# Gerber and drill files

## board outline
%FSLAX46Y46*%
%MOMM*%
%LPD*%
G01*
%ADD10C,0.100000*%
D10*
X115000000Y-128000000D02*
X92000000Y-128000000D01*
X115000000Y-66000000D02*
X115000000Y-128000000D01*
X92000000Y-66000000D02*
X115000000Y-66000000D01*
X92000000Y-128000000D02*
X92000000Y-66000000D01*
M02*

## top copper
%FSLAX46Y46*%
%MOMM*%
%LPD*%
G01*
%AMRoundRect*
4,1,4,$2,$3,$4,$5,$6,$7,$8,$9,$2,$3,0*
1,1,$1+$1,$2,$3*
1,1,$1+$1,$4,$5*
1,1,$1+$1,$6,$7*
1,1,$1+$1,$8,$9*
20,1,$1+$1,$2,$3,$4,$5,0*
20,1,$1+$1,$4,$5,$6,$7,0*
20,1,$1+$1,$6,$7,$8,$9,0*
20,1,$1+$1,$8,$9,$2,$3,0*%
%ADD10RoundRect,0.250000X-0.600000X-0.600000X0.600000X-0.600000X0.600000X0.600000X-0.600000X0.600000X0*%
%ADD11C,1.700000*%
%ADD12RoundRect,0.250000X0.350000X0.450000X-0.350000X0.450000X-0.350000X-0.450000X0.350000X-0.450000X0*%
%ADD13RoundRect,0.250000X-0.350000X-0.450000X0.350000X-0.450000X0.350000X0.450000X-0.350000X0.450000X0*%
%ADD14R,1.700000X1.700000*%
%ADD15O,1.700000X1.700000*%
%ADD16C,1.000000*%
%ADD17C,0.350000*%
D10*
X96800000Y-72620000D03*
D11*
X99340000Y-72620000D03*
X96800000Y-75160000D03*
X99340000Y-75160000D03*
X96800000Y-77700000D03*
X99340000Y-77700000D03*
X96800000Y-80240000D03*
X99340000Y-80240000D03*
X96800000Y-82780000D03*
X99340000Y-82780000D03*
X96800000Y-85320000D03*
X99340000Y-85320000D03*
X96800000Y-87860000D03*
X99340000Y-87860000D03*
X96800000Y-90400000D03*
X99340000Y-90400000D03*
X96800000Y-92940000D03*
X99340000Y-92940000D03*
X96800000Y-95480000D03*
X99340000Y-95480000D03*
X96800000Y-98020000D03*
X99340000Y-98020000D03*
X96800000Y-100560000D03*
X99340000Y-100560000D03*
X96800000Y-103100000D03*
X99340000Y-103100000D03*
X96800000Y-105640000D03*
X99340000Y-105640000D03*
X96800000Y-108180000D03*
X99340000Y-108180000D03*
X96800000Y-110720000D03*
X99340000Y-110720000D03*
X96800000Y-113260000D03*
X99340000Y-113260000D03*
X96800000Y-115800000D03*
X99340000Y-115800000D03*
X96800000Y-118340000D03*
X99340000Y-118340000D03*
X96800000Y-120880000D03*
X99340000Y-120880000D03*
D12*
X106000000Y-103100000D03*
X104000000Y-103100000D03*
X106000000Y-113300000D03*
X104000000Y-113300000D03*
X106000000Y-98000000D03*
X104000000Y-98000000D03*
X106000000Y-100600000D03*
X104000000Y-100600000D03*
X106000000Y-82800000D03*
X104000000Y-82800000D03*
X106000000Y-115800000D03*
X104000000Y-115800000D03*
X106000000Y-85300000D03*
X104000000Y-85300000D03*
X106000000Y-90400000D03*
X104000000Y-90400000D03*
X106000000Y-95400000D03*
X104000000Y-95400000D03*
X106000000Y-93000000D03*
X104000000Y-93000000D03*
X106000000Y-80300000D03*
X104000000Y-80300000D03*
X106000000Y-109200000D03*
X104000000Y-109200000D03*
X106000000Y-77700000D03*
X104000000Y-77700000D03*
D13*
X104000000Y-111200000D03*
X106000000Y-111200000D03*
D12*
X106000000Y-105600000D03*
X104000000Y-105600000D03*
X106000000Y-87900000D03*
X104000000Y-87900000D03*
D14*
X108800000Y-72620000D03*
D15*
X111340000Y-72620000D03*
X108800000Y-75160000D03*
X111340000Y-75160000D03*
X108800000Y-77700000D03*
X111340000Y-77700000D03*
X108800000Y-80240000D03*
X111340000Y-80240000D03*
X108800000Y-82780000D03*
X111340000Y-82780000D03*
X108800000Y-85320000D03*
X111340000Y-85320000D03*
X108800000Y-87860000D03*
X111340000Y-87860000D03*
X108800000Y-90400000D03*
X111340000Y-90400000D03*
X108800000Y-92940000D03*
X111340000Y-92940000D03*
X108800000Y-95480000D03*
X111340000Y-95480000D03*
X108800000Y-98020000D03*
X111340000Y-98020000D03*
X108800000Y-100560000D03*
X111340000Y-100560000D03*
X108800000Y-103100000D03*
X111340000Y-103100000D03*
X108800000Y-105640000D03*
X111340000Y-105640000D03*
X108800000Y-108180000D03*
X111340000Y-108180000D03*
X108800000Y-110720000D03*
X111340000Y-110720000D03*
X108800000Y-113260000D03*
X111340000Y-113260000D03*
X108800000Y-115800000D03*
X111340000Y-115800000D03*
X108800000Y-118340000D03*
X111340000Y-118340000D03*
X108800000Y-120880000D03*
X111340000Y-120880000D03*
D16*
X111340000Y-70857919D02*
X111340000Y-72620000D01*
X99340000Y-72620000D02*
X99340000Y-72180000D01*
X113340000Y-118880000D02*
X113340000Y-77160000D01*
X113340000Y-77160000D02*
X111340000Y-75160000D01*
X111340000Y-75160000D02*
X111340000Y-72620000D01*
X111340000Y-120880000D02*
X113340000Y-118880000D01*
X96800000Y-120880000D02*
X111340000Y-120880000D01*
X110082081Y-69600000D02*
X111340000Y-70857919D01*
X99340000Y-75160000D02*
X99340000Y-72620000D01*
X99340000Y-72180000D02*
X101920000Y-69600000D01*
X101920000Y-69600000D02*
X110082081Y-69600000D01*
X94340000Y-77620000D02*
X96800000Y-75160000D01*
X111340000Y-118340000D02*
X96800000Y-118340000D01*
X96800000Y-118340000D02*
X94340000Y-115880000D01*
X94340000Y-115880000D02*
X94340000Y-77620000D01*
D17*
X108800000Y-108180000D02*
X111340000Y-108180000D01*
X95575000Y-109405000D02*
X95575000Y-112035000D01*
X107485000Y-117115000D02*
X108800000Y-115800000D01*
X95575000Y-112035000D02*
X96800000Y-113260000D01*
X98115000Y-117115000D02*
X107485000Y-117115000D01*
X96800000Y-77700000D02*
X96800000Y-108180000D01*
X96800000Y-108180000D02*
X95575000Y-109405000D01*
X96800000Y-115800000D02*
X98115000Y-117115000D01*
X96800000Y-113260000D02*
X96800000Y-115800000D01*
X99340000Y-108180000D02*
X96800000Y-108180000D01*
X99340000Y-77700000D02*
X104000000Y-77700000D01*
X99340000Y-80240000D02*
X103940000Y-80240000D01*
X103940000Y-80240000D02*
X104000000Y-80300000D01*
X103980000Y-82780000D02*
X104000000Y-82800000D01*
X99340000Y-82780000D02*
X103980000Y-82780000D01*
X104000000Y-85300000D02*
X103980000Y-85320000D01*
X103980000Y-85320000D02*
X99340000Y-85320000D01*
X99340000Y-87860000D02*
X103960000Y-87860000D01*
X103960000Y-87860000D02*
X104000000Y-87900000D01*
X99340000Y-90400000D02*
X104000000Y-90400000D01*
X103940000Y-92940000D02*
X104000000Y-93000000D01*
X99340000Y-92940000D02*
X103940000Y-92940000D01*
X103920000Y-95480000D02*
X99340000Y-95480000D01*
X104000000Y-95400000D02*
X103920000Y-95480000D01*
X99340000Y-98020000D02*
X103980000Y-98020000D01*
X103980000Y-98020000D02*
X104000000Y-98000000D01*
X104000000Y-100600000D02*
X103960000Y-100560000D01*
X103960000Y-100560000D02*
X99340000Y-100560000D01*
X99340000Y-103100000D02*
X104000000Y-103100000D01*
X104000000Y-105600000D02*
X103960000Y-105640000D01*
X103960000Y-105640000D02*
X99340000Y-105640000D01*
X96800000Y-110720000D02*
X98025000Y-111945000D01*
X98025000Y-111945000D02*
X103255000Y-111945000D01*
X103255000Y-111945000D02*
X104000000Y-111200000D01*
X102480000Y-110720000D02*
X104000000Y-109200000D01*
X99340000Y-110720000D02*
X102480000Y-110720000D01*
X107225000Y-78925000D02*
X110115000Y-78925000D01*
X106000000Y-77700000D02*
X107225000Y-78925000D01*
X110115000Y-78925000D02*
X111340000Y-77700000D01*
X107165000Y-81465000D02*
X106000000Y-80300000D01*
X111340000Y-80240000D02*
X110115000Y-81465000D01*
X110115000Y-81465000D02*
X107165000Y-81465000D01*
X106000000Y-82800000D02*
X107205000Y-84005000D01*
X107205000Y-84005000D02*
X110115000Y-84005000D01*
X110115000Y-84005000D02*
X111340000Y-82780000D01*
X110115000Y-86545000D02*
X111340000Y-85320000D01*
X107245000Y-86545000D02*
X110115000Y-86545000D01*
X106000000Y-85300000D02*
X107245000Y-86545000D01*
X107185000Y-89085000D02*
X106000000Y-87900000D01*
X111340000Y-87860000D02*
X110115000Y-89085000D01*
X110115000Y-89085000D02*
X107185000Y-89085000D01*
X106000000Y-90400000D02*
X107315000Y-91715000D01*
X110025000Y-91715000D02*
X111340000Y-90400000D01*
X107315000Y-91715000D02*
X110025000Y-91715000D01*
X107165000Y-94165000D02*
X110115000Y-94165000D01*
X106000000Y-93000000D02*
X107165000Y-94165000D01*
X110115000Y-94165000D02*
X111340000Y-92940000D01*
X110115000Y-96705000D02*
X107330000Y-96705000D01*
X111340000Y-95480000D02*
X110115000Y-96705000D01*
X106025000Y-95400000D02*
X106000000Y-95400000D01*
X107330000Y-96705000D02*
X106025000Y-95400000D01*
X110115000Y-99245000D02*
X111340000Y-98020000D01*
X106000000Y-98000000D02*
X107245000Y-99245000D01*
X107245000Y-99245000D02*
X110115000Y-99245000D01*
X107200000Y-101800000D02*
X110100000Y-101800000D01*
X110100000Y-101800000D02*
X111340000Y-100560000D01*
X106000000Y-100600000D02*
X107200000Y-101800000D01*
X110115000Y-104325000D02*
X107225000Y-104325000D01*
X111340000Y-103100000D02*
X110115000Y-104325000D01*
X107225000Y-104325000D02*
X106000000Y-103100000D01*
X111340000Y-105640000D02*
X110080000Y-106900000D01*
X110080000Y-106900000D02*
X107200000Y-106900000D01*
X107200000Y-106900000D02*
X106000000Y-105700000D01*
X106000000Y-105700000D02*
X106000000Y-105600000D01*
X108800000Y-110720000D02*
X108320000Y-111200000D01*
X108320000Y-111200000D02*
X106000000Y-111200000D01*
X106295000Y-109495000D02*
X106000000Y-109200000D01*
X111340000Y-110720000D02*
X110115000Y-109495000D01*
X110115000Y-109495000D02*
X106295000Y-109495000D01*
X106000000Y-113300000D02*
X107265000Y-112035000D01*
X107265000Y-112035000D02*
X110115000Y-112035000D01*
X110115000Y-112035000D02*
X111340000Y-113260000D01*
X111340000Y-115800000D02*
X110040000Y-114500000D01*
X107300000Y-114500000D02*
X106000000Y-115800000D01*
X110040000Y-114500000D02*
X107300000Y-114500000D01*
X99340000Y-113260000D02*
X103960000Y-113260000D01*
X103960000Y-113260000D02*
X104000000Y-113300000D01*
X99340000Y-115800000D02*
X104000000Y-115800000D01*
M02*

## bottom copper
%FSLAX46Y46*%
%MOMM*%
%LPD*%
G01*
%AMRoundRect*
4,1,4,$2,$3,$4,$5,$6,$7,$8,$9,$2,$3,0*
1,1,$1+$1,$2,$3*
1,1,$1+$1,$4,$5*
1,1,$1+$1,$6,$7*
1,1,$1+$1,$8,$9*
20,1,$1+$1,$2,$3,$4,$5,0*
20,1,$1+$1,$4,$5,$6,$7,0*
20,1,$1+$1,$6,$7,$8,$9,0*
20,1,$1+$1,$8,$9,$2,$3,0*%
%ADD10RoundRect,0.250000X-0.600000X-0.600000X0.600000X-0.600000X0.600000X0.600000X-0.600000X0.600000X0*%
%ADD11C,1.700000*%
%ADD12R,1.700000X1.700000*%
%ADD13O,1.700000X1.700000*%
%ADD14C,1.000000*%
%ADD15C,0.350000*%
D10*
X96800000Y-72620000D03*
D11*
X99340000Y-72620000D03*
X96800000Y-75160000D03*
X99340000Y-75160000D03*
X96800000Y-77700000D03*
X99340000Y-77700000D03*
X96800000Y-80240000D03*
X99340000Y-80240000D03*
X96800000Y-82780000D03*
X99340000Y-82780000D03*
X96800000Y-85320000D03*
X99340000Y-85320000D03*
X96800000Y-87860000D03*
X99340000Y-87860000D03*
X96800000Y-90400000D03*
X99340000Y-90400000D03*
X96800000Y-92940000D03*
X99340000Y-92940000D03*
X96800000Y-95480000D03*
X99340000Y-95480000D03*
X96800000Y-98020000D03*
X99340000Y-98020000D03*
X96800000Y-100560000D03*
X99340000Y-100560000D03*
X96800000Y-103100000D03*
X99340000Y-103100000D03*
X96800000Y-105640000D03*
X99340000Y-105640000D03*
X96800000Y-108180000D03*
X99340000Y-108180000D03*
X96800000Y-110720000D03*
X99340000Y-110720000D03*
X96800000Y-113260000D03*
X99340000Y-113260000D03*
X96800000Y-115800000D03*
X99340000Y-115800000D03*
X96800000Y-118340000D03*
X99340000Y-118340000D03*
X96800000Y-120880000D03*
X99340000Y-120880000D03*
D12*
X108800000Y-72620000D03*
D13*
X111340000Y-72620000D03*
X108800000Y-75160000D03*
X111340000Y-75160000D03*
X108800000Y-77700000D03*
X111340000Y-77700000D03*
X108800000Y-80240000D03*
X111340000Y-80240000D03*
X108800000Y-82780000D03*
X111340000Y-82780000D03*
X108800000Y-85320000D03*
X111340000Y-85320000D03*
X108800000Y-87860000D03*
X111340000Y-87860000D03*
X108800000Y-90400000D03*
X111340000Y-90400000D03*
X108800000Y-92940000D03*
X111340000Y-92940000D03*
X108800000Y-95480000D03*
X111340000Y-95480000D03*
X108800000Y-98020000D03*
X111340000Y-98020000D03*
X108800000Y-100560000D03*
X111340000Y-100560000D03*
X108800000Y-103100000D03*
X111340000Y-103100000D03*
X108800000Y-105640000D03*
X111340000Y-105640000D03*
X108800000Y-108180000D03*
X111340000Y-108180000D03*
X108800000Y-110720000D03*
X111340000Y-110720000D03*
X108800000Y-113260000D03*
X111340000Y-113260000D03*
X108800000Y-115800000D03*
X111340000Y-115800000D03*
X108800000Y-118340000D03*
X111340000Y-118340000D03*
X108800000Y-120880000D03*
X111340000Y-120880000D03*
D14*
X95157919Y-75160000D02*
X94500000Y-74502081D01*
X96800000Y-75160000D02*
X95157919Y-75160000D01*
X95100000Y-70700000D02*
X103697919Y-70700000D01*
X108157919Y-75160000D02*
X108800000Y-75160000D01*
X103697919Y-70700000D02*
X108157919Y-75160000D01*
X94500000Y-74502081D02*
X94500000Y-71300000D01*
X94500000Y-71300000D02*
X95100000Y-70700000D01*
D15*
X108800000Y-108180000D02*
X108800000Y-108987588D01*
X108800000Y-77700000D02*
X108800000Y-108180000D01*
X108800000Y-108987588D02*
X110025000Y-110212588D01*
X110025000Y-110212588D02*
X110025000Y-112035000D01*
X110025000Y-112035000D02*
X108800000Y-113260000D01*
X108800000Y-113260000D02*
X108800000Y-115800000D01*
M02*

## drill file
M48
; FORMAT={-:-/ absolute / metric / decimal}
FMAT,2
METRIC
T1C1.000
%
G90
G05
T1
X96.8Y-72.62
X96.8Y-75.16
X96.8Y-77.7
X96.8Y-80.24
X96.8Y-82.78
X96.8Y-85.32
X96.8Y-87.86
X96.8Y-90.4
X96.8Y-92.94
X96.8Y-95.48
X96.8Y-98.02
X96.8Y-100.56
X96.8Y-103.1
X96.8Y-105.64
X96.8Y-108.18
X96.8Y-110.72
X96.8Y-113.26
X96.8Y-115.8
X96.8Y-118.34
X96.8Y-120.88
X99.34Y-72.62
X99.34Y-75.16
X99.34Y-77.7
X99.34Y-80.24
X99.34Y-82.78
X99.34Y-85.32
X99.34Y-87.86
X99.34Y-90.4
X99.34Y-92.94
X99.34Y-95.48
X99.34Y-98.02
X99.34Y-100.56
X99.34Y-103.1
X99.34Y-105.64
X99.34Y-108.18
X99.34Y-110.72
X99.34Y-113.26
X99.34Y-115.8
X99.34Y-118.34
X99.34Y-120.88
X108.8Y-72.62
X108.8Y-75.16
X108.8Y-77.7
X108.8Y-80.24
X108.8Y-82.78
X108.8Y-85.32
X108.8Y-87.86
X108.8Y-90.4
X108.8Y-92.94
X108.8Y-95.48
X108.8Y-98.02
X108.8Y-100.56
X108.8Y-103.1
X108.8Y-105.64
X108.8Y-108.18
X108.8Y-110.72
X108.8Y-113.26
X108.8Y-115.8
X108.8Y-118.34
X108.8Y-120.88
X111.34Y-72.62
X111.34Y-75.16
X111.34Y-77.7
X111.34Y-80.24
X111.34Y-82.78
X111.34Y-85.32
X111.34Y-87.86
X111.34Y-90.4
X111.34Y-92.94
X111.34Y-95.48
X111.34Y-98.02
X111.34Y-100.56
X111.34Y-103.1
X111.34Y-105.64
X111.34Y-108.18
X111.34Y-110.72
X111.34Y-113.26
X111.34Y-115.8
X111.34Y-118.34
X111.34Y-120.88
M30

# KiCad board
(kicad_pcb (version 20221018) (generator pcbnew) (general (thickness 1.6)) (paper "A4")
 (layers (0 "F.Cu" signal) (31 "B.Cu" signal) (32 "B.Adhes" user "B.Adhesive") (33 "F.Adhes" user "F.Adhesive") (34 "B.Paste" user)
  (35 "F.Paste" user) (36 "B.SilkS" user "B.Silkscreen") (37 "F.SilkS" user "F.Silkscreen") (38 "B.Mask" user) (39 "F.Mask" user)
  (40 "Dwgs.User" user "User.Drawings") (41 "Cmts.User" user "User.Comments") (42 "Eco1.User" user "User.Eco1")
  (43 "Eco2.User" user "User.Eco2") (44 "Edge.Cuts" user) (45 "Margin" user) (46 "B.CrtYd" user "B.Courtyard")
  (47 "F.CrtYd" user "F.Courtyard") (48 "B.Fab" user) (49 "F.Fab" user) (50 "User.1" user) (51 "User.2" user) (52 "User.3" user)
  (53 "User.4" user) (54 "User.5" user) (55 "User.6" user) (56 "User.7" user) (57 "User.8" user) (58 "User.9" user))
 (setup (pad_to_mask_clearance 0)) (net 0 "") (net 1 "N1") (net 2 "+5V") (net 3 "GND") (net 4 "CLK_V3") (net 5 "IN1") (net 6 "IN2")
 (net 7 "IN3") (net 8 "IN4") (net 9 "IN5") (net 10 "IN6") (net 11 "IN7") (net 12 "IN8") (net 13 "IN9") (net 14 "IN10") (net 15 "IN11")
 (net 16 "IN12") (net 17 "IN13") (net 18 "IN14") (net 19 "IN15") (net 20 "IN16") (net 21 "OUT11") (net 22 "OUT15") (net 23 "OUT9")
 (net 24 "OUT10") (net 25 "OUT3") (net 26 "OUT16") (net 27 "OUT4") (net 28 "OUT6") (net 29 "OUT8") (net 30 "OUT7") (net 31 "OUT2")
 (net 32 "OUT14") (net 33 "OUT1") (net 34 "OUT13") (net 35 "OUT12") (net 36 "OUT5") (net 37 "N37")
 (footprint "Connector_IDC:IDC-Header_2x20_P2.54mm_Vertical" (layer "F.Cu") (at 96.8 72.62)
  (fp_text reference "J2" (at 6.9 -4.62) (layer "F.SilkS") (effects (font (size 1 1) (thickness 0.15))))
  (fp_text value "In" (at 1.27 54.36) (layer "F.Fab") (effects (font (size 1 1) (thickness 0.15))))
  (pad "1" thru_hole roundrect (at 0 0) (size 1.7 1.7) (drill 1) (layers "*.Cu" "*.Mask") (roundrect_rratio 0.1470588235) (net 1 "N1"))
  (pad "2" thru_hole circle (at 2.54 0) (size 1.7 1.7) (drill 1) (layers "*.Cu" "*.Mask") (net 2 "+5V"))
  (pad "3" thru_hole circle (at 0 2.54) (size 1.7 1.7) (drill 1) (layers "*.Cu" "*.Mask") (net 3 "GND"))
  (pad "4" thru_hole circle (at 2.54 2.54) (size 1.7 1.7) (drill 1) (layers "*.Cu" "*.Mask") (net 2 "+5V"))
  (pad "5" thru_hole circle (at 0 5.08) (size 1.7 1.7) (drill 1) (layers "*.Cu" "*.Mask") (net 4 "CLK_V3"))
  (pad "6" thru_hole circle (at 2.54 5.08) (size 1.7 1.7) (drill 1) (layers "*.Cu" "*.Mask") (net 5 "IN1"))
  (pad "7" thru_hole circle (at 0 7.62) (size 1.7 1.7) (drill 1) (layers "*.Cu" "*.Mask") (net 4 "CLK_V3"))
  (pad "8" thru_hole circle (at 2.54 7.62) (size 1.7 1.7) (drill 1) (layers "*.Cu" "*.Mask") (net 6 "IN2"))
  (pad "9" thru_hole circle (at 0 10.16) (size 1.7 1.7) (drill 1) (layers "*.Cu" "*.Mask") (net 4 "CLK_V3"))
  (pad "10" thru_hole circle (at 2.54 10.16) (size 1.7 1.7) (drill 1) (layers "*.Cu" "*.Mask") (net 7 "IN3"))
  (pad "11" thru_hole circle (at 0 12.7) (size 1.7 1.7) (drill 1) (layers "*.Cu" "*.Mask") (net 4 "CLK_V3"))
  (pad "12" thru_hole circle (at 2.54 12.7) (size 1.7 1.7) (drill 1) (layers "*.Cu" "*.Mask") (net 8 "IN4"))
  (pad "13" thru_hole circle (at 0 15.24) (size 1.7 1.7) (drill 1) (layers "*.Cu" "*.Mask") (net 4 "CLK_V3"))
  (pad "14" thru_hole circle (at 2.54 15.24) (size 1.7 1.7) (drill 1) (layers "*.Cu" "*.Mask") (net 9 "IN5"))
  (pad "15" thru_hole circle (at 0 17.78) (size 1.7 1.7) (drill 1) (layers "*.Cu" "*.Mask") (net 4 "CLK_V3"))
  (pad "16" thru_hole circle (at 2.54 17.78) (size 1.7 1.7) (drill 1) (layers "*.Cu" "*.Mask") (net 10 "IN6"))
  (pad "17" thru_hole circle (at 0 20.32) (size 1.7 1.7) (drill 1) (layers "*.Cu" "*.Mask") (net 4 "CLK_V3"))
  (pad "18" thru_hole circle (at 2.54 20.32) (size 1.7 1.7) (drill 1) (layers "*.Cu" "*.Mask") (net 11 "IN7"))
  (pad "19" thru_hole circle (at 0 22.86) (size 1.7 1.7) (drill 1) (layers "*.Cu" "*.Mask") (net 4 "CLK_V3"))
  (pad "20" thru_hole circle (at 2.54 22.86) (size 1.7 1.7) (drill 1) (layers "*.Cu" "*.Mask") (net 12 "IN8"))
  (pad "21" thru_hole circle (at 0 25.4) (size 1.7 1.7) (drill 1) (layers "*.Cu" "*.Mask") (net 4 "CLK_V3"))
  (pad "22" thru_hole circle (at 2.54 25.4) (size 1.7 1.7) (drill 1) (layers "*.Cu" "*.Mask") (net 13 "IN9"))
  (pad "23" thru_hole circle (at 0 27.94) (size 1.7 1.7) (drill 1) (layers "*.Cu" "*.Mask") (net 4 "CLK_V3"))
  (pad "24" thru_hole circle (at 2.54 27.94) (size 1.7 1.7) (drill 1) (layers "*.Cu" "*.Mask") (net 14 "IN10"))
  (pad "25" thru_hole circle (at 0 30.48) (size 1.7 1.7) (drill 1) (layers "*.Cu" "*.Mask") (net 4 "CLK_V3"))
  (pad "26" thru_hole circle (at 2.54 30.48) (size 1.7 1.7) (drill 1) (layers "*.Cu" "*.Mask") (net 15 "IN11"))
  (pad "27" thru_hole circle (at 0 33.02) (size 1.7 1.7) (drill 1) (layers "*.Cu" "*.Mask") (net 4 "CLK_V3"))
  (pad "28" thru_hole circle (at 2.54 33.02) (size 1.7 1.7) (drill 1) (layers "*.Cu" "*.Mask") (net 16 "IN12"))
  (pad "29" thru_hole circle (at 0 35.56) (size 1.7 1.7) (drill 1) (layers "*.Cu" "*.Mask") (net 4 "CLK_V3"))
  (pad "30" thru_hole circle (at 2.54 35.56) (size 1.7 1.7) (drill 1) (layers "*.Cu" "*.Mask") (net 4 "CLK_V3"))
  (pad "31" thru_hole circle (at 0 38.1) (size 1.7 1.7) (drill 1) (layers "*.Cu" "*.Mask") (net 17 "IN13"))
  (pad "32" thru_hole circle (at 2.54 38.1) (size 1.7 1.7) (drill 1) (layers "*.Cu" "*.Mask") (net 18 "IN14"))
  (pad "33" thru_hole circle (at 0 40.64) (size 1.7 1.7) (drill 1) (layers "*.Cu" "*.Mask") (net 4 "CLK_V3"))
  (pad "34" thru_hole circle (at 2.54 40.64) (size 1.7 1.7) (drill 1) (layers "*.Cu" "*.Mask") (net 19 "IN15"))
  (pad "35" thru_hole circle (at 0 43.18) (size 1.7 1.7) (drill 1) (layers "*.Cu" "*.Mask") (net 4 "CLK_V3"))
  (pad "36" thru_hole circle (at 2.54 43.18) (size 1.7 1.7) (drill 1) (layers "*.Cu" "*.Mask") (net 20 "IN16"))
  (pad "37" thru_hole circle (at 0 45.72) (size 1.7 1.7) (drill 1) (layers "*.Cu" "*.Mask") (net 3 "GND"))
  (pad "38" thru_hole circle (at 2.54 45.72) (size 1.7 1.7) (drill 1) (layers "*.Cu" "*.Mask") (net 3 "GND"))
  (pad "39" thru_hole circle (at 0 48.26) (size 1.7 1.7) (drill 1) (layers "*.Cu" "*.Mask") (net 2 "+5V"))
  (pad "40" thru_hole circle (at 2.54 48.26) (size 1.7 1.7) (drill 1) (layers "*.Cu" "*.Mask") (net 2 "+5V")))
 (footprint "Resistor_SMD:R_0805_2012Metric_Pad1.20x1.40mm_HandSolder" (layer "F.Cu") (at 105 103.1 180)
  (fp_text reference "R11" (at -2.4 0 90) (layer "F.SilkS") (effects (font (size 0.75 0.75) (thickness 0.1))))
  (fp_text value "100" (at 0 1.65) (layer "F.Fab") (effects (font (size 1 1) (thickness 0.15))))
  (pad "1" smd roundrect (at -1 0 180) (size 1.2 1.4) (layers "F.Cu" "F.Paste" "F.Mask") (roundrect_rratio 0.2083333333) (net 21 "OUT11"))
  (pad "2" smd roundrect (at 1 0 180) (size 1.2 1.4) (layers "F.Cu" "F.Paste" "F.Mask") (roundrect_rratio 0.2083333333) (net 15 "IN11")))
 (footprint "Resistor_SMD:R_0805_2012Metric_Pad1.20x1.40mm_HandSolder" (layer "F.Cu") (at 105 113.3 180)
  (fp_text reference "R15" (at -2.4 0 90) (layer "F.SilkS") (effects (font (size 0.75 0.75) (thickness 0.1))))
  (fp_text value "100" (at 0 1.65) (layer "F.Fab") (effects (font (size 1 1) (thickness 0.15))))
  (pad "1" smd roundrect (at -1 0 180) (size 1.2 1.4) (layers "F.Cu" "F.Paste" "F.Mask") (roundrect_rratio 0.2083333333) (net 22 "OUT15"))
  (pad "2" smd roundrect (at 1 0 180) (size 1.2 1.4) (layers "F.Cu" "F.Paste" "F.Mask") (roundrect_rratio 0.2083333333) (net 19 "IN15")))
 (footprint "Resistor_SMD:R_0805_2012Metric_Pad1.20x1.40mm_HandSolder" (layer "F.Cu") (at 105 98 180)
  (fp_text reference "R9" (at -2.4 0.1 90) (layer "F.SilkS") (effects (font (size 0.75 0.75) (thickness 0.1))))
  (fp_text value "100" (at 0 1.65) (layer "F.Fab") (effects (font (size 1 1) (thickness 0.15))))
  (pad "1" smd roundrect (at -1 0 180) (size 1.2 1.4) (layers "F.Cu" "F.Paste" "F.Mask") (roundrect_rratio 0.2083333333) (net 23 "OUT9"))
  (pad "2" smd roundrect (at 1 0 180) (size 1.2 1.4) (layers "F.Cu" "F.Paste" "F.Mask") (roundrect_rratio 0.2083333333) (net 13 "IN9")))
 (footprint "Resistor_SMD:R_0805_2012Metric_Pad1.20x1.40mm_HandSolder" (layer "F.Cu") (at 105 100.6 180)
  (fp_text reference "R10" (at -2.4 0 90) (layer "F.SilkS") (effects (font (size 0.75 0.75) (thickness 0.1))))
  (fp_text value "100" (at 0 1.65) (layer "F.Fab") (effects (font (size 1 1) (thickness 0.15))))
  (pad "1" smd roundrect (at -1 0 180) (size 1.2 1.4) (layers "F.Cu" "F.Paste" "F.Mask") (roundrect_rratio 0.2083333333) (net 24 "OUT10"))
  (pad "2" smd roundrect (at 1 0 180) (size 1.2 1.4) (layers "F.Cu" "F.Paste" "F.Mask") (roundrect_rratio 0.2083333333) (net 14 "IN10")))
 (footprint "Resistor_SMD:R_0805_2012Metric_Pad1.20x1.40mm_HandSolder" (layer "F.Cu") (at 105 82.8 180)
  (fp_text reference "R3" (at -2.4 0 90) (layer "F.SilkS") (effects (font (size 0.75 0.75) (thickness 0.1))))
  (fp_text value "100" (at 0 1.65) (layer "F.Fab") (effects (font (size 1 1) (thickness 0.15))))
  (pad "1" smd roundrect (at -1 0 180) (size 1.2 1.4) (layers "F.Cu" "F.Paste" "F.Mask") (roundrect_rratio 0.2083333333) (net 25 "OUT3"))
  (pad "2" smd roundrect (at 1 0 180) (size 1.2 1.4) (layers "F.Cu" "F.Paste" "F.Mask") (roundrect_rratio 0.2083333333) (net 7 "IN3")))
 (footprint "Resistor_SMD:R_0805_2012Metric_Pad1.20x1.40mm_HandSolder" (layer "F.Cu") (at 105 115.8 180)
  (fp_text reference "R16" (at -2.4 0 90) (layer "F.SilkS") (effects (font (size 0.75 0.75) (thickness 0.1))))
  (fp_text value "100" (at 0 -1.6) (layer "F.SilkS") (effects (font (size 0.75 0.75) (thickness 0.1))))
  (pad "1" smd roundrect (at -1 0 180) (size 1.2 1.4) (layers "F.Cu" "F.Paste" "F.Mask") (roundrect_rratio 0.2083333333) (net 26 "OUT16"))
  (pad "2" smd roundrect (at 1 0 180) (size 1.2 1.4) (layers "F.Cu" "F.Paste" "F.Mask") (roundrect_rratio 0.2083333333) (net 20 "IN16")))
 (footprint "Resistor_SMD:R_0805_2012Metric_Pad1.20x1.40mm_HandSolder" (layer "F.Cu") (at 105 85.3 180)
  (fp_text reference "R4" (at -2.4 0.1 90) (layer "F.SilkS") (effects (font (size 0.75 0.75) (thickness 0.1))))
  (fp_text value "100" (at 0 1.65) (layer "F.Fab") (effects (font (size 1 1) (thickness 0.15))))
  (pad "1" smd roundrect (at -1 0 180) (size 1.2 1.4) (layers "F.Cu" "F.Paste" "F.Mask") (roundrect_rratio 0.2083333333) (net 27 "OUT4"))
  (pad "2" smd roundrect (at 1 0 180) (size 1.2 1.4) (layers "F.Cu" "F.Paste" "F.Mask") (roundrect_rratio 0.2083333333) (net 8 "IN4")))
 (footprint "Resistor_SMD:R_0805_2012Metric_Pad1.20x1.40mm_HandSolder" (layer "F.Cu") (at 105 90.4 180)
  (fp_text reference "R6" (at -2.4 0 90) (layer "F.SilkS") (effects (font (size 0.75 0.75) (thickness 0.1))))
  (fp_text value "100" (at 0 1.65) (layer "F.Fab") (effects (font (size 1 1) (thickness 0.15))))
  (pad "1" smd roundrect (at -1 0 180) (size 1.2 1.4) (layers "F.Cu" "F.Paste" "F.Mask") (roundrect_rratio 0.2083333333) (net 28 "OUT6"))
  (pad "2" smd roundrect (at 1 0 180) (size 1.2 1.4) (layers "F.Cu" "F.Paste" "F.Mask") (roundrect_rratio 0.2083333333) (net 10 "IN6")))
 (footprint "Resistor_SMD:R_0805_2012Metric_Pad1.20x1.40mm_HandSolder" (layer "F.Cu") (at 105 95.4 180)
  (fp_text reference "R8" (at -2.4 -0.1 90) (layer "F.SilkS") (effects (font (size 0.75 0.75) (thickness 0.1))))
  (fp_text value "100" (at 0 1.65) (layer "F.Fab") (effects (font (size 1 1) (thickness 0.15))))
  (pad "1" smd roundrect (at -1 0 180) (size 1.2 1.4) (layers "F.Cu" "F.Paste" "F.Mask") (roundrect_rratio 0.2083333333) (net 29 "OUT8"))
  (pad "2" smd roundrect (at 1 0 180) (size 1.2 1.4) (layers "F.Cu" "F.Paste" "F.Mask") (roundrect_rratio 0.2083333333) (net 12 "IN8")))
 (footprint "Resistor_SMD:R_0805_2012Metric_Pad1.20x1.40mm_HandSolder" (layer "F.Cu") (at 105 93 180)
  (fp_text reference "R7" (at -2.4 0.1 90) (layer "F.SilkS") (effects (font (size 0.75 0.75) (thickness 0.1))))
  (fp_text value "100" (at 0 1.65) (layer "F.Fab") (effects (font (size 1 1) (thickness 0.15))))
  (pad "1" smd roundrect (at -1 0 180) (size 1.2 1.4) (layers "F.Cu" "F.Paste" "F.Mask") (roundrect_rratio 0.2083333333) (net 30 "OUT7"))
  (pad "2" smd roundrect (at 1 0 180) (size 1.2 1.4) (layers "F.Cu" "F.Paste" "F.Mask") (roundrect_rratio 0.2083333333) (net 11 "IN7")))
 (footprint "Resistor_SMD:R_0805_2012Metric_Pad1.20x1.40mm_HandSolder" (layer "F.Cu") (at 105 80.3 180)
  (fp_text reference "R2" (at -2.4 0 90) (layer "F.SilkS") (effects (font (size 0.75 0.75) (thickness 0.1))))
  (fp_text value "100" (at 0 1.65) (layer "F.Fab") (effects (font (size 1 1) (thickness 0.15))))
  (pad "1" smd roundrect (at -1 0 180) (size 1.2 1.4) (layers "F.Cu" "F.Paste" "F.Mask") (roundrect_rratio 0.2083333333) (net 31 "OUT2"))
  (pad "2" smd roundrect (at 1 0 180) (size 1.2 1.4) (layers "F.Cu" "F.Paste" "F.Mask") (roundrect_rratio 0.2083333333) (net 6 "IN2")))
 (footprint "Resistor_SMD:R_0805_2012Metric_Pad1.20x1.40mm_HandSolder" (layer "F.Cu") (at 105 109.2 180)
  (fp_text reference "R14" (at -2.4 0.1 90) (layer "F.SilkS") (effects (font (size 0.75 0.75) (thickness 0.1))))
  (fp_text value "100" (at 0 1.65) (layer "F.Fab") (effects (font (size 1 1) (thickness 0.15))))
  (pad "1" smd roundrect (at -1 0 180) (size 1.2 1.4) (layers "F.Cu" "F.Paste" "F.Mask") (roundrect_rratio 0.2083333333) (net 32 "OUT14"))
  (pad "2" smd roundrect (at 1 0 180) (size 1.2 1.4) (layers "F.Cu" "F.Paste" "F.Mask") (roundrect_rratio 0.2083333333) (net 18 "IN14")))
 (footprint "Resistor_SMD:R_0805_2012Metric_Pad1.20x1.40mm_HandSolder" (layer "F.Cu") (at 105 77.7 180)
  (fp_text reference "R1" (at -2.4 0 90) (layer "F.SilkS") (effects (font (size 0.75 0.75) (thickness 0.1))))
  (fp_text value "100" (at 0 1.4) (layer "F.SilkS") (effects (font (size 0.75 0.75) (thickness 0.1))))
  (pad "1" smd roundrect (at -1 0 180) (size 1.2 1.4) (layers "F.Cu" "F.Paste" "F.Mask") (roundrect_rratio 0.2083333333) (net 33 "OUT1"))
  (pad "2" smd roundrect (at 1 0 180) (size 1.2 1.4) (layers "F.Cu" "F.Paste" "F.Mask") (roundrect_rratio 0.2083333333) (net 5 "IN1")))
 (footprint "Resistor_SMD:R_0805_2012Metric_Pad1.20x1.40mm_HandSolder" (layer "F.Cu") (at 105 111.2)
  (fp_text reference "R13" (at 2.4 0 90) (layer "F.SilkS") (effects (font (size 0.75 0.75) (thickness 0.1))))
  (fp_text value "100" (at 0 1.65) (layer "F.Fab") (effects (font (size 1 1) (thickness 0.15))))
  (pad "1" smd roundrect (at -1 0) (size 1.2 1.4) (layers "F.Cu" "F.Paste" "F.Mask") (roundrect_rratio 0.2083333333) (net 17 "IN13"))
  (pad "2" smd roundrect (at 1 0) (size 1.2 1.4) (layers "F.Cu" "F.Paste" "F.Mask") (roundrect_rratio 0.2083333333) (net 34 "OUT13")))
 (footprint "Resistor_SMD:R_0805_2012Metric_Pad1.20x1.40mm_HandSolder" (layer "F.Cu") (at 105 105.6 180)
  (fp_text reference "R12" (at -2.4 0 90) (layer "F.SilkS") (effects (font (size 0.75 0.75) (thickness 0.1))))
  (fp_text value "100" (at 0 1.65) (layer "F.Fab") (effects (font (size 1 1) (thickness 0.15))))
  (pad "1" smd roundrect (at -1 0 180) (size 1.2 1.4) (layers "F.Cu" "F.Paste" "F.Mask") (roundrect_rratio 0.2083333333) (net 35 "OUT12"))
  (pad "2" smd roundrect (at 1 0 180) (size 1.2 1.4) (layers "F.Cu" "F.Paste" "F.Mask") (roundrect_rratio 0.2083333333) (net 16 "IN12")))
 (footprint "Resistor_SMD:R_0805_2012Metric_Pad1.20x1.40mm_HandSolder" (layer "F.Cu") (at 105 87.9 180)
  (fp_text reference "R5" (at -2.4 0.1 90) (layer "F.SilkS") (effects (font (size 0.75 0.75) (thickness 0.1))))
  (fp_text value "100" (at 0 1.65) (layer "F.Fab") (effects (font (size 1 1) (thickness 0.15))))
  (pad "1" smd roundrect (at -1 0 180) (size 1.2 1.4) (layers "F.Cu" "F.Paste" "F.Mask") (roundrect_rratio 0.2083333333) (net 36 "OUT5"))
  (pad "2" smd roundrect (at 1 0 180) (size 1.2 1.4) (layers "F.Cu" "F.Paste" "F.Mask") (roundrect_rratio 0.2083333333) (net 9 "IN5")))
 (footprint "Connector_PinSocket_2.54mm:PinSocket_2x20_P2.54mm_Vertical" (layer "B.Cu") (at 108.8 72.62 180)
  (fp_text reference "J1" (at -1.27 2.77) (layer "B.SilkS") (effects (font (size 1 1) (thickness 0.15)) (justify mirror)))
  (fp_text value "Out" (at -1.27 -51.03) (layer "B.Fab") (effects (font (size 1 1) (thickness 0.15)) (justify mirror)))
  (pad "1" thru_hole rect (at 0 0 180) (size 1.7 1.7) (drill 1) (layers "*.Cu" "*.Mask") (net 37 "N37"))
  (pad "2" thru_hole oval (at -2.54 0 180) (size 1.7 1.7) (drill 1) (layers "*.Cu" "*.Mask") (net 2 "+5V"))
  (pad "3" thru_hole oval (at 0 -2.54 180) (size 1.7 1.7) (drill 1) (layers "*.Cu" "*.Mask") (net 3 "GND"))
  (pad "4" thru_hole oval (at -2.54 -2.54 180) (size 1.7 1.7) (drill 1) (layers "*.Cu" "*.Mask") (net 2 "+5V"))
  (pad "5" thru_hole oval (at 0 -5.08 180) (size 1.7 1.7) (drill 1) (layers "*.Cu" "*.Mask") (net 4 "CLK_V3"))
  (pad "6" thru_hole oval (at -2.54 -5.08 180) (size 1.7 1.7) (drill 1) (layers "*.Cu" "*.Mask") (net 33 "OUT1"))
  (pad "7" thru_hole oval (at 0 -7.62 180) (size 1.7 1.7) (drill 1) (layers "*.Cu" "*.Mask") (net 4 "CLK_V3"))
  (pad "8" thru_hole oval (at -2.54 -7.62 180) (size 1.7 1.7) (drill 1) (layers "*.Cu" "*.Mask") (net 31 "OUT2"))
  (pad "9" thru_hole oval (at 0 -10.16 180) (size 1.7 1.7) (drill 1) (layers "*.Cu" "*.Mask") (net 4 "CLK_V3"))
  (pad "10" thru_hole oval (at -2.54 -10.16 180) (size 1.7 1.7) (drill 1) (layers "*.Cu" "*.Mask") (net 25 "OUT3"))
  (pad "11" thru_hole oval (at 0 -12.7 180) (size 1.7 1.7) (drill 1) (layers "*.Cu" "*.Mask") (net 4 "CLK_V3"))
  (pad "12" thru_hole oval (at -2.54 -12.7 180) (size 1.7 1.7) (drill 1) (layers "*.Cu" "*.Mask") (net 27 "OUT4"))
  (pad "13" thru_hole oval (at 0 -15.24 180) (size 1.7 1.7) (drill 1) (layers "*.Cu" "*.Mask") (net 4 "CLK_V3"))
  (pad "14" thru_hole oval (at -2.54 -15.24 180) (size 1.7 1.7) (drill 1) (layers "*.Cu" "*.Mask") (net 36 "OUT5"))
  (pad "15" thru_hole oval (at 0 -17.78 180) (size 1.7 1.7) (drill 1) (layers "*.Cu" "*.Mask") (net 4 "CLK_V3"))
  (pad "16" thru_hole oval (at -2.54 -17.78 180) (size 1.7 1.7) (drill 1) (layers "*.Cu" "*.Mask") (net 28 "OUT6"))
  (pad "17" thru_hole oval (at 0 -20.32 180) (size 1.7 1.7) (drill 1) (layers "*.Cu" "*.Mask") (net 4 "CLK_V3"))
  (pad "18" thru_hole oval (at -2.54 -20.32 180) (size 1.7 1.7) (drill 1) (layers "*.Cu" "*.Mask") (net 30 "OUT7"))
  (pad "19" thru_hole oval (at 0 -22.86 180) (size 1.7 1.7) (drill 1) (layers "*.Cu" "*.Mask") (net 4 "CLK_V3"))
  (pad "20" thru_hole oval (at -2.54 -22.86 180) (size 1.7 1.7) (drill 1) (layers "*.Cu" "*.Mask") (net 29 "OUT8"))
  (pad "21" thru_hole oval (at 0 -25.4 180) (size 1.7 1.7) (drill 1) (layers "*.Cu" "*.Mask") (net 4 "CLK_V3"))
  (pad "22" thru_hole oval (at -2.54 -25.4 180) (size 1.7 1.7) (drill 1) (layers "*.Cu" "*.Mask") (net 23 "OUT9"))
  (pad "23" thru_hole oval (at 0 -27.94 180) (size 1.7 1.7) (drill 1) (layers "*.Cu" "*.Mask") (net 4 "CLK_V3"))
  (pad "24" thru_hole oval (at -2.54 -27.94 180) (size 1.7 1.7) (drill 1) (layers "*.Cu" "*.Mask") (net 24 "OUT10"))
  (pad "25" thru_hole oval (at 0 -30.48 180) (size 1.7 1.7) (drill 1) (layers "*.Cu" "*.Mask") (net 4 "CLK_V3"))
  (pad "26" thru_hole oval (at -2.54 -30.48 180) (size 1.7 1.7) (drill 1) (layers "*.Cu" "*.Mask") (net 21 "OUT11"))
  (pad "27" thru_hole oval (at 0 -33.02 180) (size 1.7 1.7) (drill 1) (layers "*.Cu" "*.Mask") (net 4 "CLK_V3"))
  (pad "28" thru_hole oval (at -2.54 -33.02 180) (size 1.7 1.7) (drill 1) (layers "*.Cu" "*.Mask") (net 35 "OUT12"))
  (pad "29" thru_hole oval (at 0 -35.56 180) (size 1.7 1.7) (drill 1) (layers "*.Cu" "*.Mask") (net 4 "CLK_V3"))
  (pad "30" thru_hole oval (at -2.54 -35.56 180) (size 1.7 1.7) (drill 1) (layers "*.Cu" "*.Mask") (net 4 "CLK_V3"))
  (pad "31" thru_hole oval (at 0 -38.1 180) (size 1.7 1.7) (drill 1) (layers "*.Cu" "*.Mask") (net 34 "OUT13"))
  (pad "32" thru_hole oval (at -2.54 -38.1 180) (size 1.7 1.7) (drill 1) (layers "*.Cu" "*.Mask") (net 32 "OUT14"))
  (pad "33" thru_hole oval (at 0 -40.64 180) (size 1.7 1.7) (drill 1) (layers "*.Cu" "*.Mask") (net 4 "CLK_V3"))
  (pad "34" thru_hole oval (at -2.54 -40.64 180) (size 1.7 1.7) (drill 1) (layers "*.Cu" "*.Mask") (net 22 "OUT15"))
  (pad "35" thru_hole oval (at 0 -43.18 180) (size 1.7 1.7) (drill 1) (layers "*.Cu" "*.Mask") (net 4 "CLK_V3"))
  (pad "36" thru_hole oval (at -2.54 -43.18 180) (size 1.7 1.7) (drill 1) (layers "*.Cu" "*.Mask") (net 26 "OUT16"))
  (pad "37" thru_hole oval (at 0 -45.72 180) (size 1.7 1.7) (drill 1) (layers "*.Cu" "*.Mask") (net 3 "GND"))
  (pad "38" thru_hole oval (at -2.54 -45.72 180) (size 1.7 1.7) (drill 1) (layers "*.Cu" "*.Mask") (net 3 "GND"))
  (pad "39" thru_hole oval (at 0 -48.26 180) (size 1.7 1.7) (drill 1) (layers "*.Cu" "*.Mask") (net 2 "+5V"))
  (pad "40" thru_hole oval (at -2.54 -48.26 180) (size 1.7 1.7) (drill 1) (layers "*.Cu" "*.Mask") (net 2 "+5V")))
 (gr_line (start 115 128) (end 92 128) (stroke (width 0.1) (type default)) (layer "Edge.Cuts"))
 (gr_line (start 115 66) (end 115 128) (stroke (width 0.1) (type default)) (layer "Edge.Cuts"))
 (gr_line (start 92 66) (end 115 66) (stroke (width 0.1) (type default)) (layer "Edge.Cuts"))
 (gr_line (start 92 128) (end 92 66) (stroke (width 0.1) (type default)) (layer "Edge.Cuts"))
 (segment (start 111.34 70.857919) (end 111.34 72.62) (width 1) (layer "F.Cu") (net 2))
 (segment (start 99.34 72.62) (end 99.34 72.18) (width 1) (layer "F.Cu") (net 2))
 (segment (start 113.34 118.88) (end 113.34 77.16) (width 1) (layer "F.Cu") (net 2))
 (segment (start 113.34 77.16) (end 111.34 75.16) (width 1) (layer "F.Cu") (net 2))
 (segment (start 111.34 75.16) (end 111.34 72.62) (width 1) (layer "F.Cu") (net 2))
 (segment (start 111.34 120.88) (end 113.34 118.88) (width 1) (layer "F.Cu") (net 2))
 (segment (start 96.8 120.88) (end 111.34 120.88) (width 1) (layer "F.Cu") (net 2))
 (segment (start 110.082081 69.6) (end 111.34 70.857919) (width 1) (layer "F.Cu") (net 2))
 (segment (start 99.34 75.16) (end 99.34 72.62) (width 1) (layer "F.Cu") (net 2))
 (segment (start 99.34 72.18) (end 101.92 69.6) (width 1) (layer "F.Cu") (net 2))
 (segment (start 101.92 69.6) (end 110.082081 69.6) (width 1) (layer "F.Cu") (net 2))
 (segment (start 94.34 77.62) (end 96.8 75.16) (width 1) (layer "F.Cu") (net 3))
 (segment (start 111.34 118.34) (end 96.8 118.34) (width 1) (layer "F.Cu") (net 3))
 (segment (start 96.8 118.34) (end 94.34 115.88) (width 1) (layer "F.Cu") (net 3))
 (segment (start 94.34 115.88) (end 94.34 77.62) (width 1) (layer "F.Cu") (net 3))
 (segment (start 95.157919 75.16) (end 94.5 74.502081) (width 1) (layer "B.Cu") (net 3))
 (segment (start 96.8 75.16) (end 95.157919 75.16) (width 1) (layer "B.Cu") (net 3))
 (segment (start 95.1 70.7) (end 103.697919 70.7) (width 1) (layer "B.Cu") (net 3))
 (segment (start 108.157919 75.16) (end 108.8 75.16) (width 1) (layer "B.Cu") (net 3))
 (segment (start 103.697919 70.7) (end 108.157919 75.16) (width 1) (layer "B.Cu") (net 3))
 (segment (start 94.5 74.502081) (end 94.5 71.3) (width 1) (layer "B.Cu") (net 3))
 (segment (start 94.5 71.3) (end 95.1 70.7) (width 1) (layer "B.Cu") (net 3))
 (segment (start 108.8 108.18) (end 111.34 108.18) (width 0.35) (layer "F.Cu") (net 4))
 (segment (start 95.575 109.405) (end 95.575 112.035) (width 0.35) (layer "F.Cu") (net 4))
 (segment (start 107.485 117.115) (end 108.8 115.8) (width 0.35) (layer "F.Cu") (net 4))
 (segment (start 95.575 112.035) (end 96.8 113.26) (width 0.35) (layer "F.Cu") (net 4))
 (segment (start 98.115 117.115) (end 107.485 117.115) (width 0.35) (layer "F.Cu") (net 4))
 (segment (start 96.8 77.7) (end 96.8 108.18) (width 0.35) (layer "F.Cu") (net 4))
 (segment (start 96.8 108.18) (end 95.575 109.405) (width 0.35) (layer "F.Cu") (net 4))
 (segment (start 96.8 115.8) (end 98.115 117.115) (width 0.35) (layer "F.Cu") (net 4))
 (segment (start 96.8 113.26) (end 96.8 115.8) (width 0.35) (layer "F.Cu") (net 4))
 (segment (start 99.34 108.18) (end 96.8 108.18) (width 0.35) (layer "F.Cu") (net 4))
 (segment (start 108.8 108.18) (end 108.8 108.987588) (width 0.35) (layer "B.Cu") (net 4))
 (segment (start 108.8 77.7) (end 108.8 108.18) (width 0.35) (layer "B.Cu") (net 4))
 (segment (start 108.8 108.987588) (end 110.025 110.212588) (width 0.35) (layer "B.Cu") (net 4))
 (segment (start 110.025 110.212588) (end 110.025 112.035) (width 0.35) (layer "B.Cu") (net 4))
 (segment (start 110.025 112.035) (end 108.8 113.26) (width 0.35) (layer "B.Cu") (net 4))
 (segment (start 108.8 113.26) (end 108.8 115.8) (width 0.35) (layer "B.Cu") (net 4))
 (segment (start 99.34 77.7) (end 104 77.7) (width 0.35) (layer "F.Cu") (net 5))
 (segment (start 99.34 80.24) (end 103.94 80.24) (width 0.35) (layer "F.Cu") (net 6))
 (segment (start 103.94 80.24) (end 104 80.3) (width 0.35) (layer "F.Cu") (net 6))
 (segment (start 103.98 82.78) (end 104 82.8) (width 0.35) (layer "F.Cu") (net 7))
 (segment (start 99.34 82.78) (end 103.98 82.78) (width 0.35) (layer "F.Cu") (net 7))
 (segment (start 104 85.3) (end 103.98 85.32) (width 0.35) (layer "F.Cu") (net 8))
 (segment (start 103.98 85.32) (end 99.34 85.32) (width 0.35) (layer "F.Cu") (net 8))
 (segment (start 99.34 87.86) (end 103.96 87.86) (width 0.35) (layer "F.Cu") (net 9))
 (segment (start 103.96 87.86) (end 104 87.9) (width 0.35) (layer "F.Cu") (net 9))
 (segment (start 99.34 90.4) (end 104 90.4) (width 0.35) (layer "F.Cu") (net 10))
 (segment (start 103.94 92.94) (end 104 93) (width 0.35) (layer "F.Cu") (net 11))
 (segment (start 99.34 92.94) (end 103.94 92.94) (width 0.35) (layer "F.Cu") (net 11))
 (segment (start 103.92 95.48) (end 99.34 95.48) (width 0.35) (layer "F.Cu") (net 12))
 (segment (start 104 95.4) (end 103.92 95.48) (width 0.35) (layer "F.Cu") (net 12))
 (segment (start 99.34 98.02) (end 103.98 98.02) (width 0.35) (layer "F.Cu") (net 13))
 (segment (start 103.98 98.02) (end 104 98) (width 0.35) (layer "F.Cu") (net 13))
 (segment (start 104 100.6) (end 103.96 100.56) (width 0.35) (layer "F.Cu") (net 14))
 (segment (start 103.96 100.56) (end 99.34 100.56) (width 0.35) (layer "F.Cu") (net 14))
 (segment (start 99.34 103.1) (end 104 103.1) (width 0.35) (layer "F.Cu") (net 15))
 (segment (start 104 105.6) (end 103.96 105.64) (width 0.35) (layer "F.Cu") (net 16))
 (segment (start 103.96 105.64) (end 99.34 105.64) (width 0.35) (layer "F.Cu") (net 16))
 (segment (start 96.8 110.72) (end 98.025 111.945) (width 0.35) (layer "F.Cu") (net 17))
 (segment (start 98.025 111.945) (end 103.255 111.945) (width 0.35) (layer "F.Cu") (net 17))
 (segment (start 103.255 111.945) (end 104 111.2) (width 0.35) (layer "F.Cu") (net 17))
 (segment (start 102.48 110.72) (end 104 109.2) (width 0.35) (layer "F.Cu") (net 18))
 (segment (start 99.34 110.72) (end 102.48 110.72) (width 0.35) (layer "F.Cu") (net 18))
 (segment (start 107.225 78.925) (end 110.115 78.925) (width 0.35) (layer "F.Cu") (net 33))
 (segment (start 106 77.7) (end 107.225 78.925) (width 0.35) (layer "F.Cu") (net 33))
 (segment (start 110.115 78.925) (end 111.34 77.7) (width 0.35) (layer "F.Cu") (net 33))
 (segment (start 107.165 81.465) (end 106 80.3) (width 0.35) (layer "F.Cu") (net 31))
 (segment (start 111.34 80.24) (end 110.115 81.465) (width 0.35) (layer "F.Cu") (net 31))
 (segment (start 110.115 81.465) (end 107.165 81.465) (width 0.35) (layer "F.Cu") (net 31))
 (segment (start 106 82.8) (end 107.205 84.005) (width 0.35) (layer "F.Cu") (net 25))
 (segment (start 107.205 84.005) (end 110.115 84.005) (width 0.35) (layer "F.Cu") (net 25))
 (segment (start 110.115 84.005) (end 111.34 82.78) (width 0.35) (layer "F.Cu") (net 25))
 (segment (start 110.115 86.545) (end 111.34 85.32) (width 0.35) (layer "F.Cu") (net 27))
 (segment (start 107.245 86.545) (end 110.115 86.545) (width 0.35) (layer "F.Cu") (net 27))
 (segment (start 106 85.3) (end 107.245 86.545) (width 0.35) (layer "F.Cu") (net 27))
 (segment (start 107.185 89.085) (end 106 87.9) (width 0.35) (layer "F.Cu") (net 36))
 (segment (start 111.34 87.86) (end 110.115 89.085) (width 0.35) (layer "F.Cu") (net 36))
 (segment (start 110.115 89.085) (end 107.185 89.085) (width 0.35) (layer "F.Cu") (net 36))
 (segment (start 106 90.4) (end 107.315 91.715) (width 0.35) (layer "F.Cu") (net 28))
 (segment (start 110.025 91.715) (end 111.34 90.4) (width 0.35) (layer "F.Cu") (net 28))
 (segment (start 107.315 91.715) (end 110.025 91.715) (width 0.35) (layer "F.Cu") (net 28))
 (segment (start 107.165 94.165) (end 110.115 94.165) (width 0.35) (layer "F.Cu") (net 30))
 (segment (start 106 93) (end 107.165 94.165) (width 0.35) (layer "F.Cu") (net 30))
 (segment (start 110.115 94.165) (end 111.34 92.94) (width 0.35) (layer "F.Cu") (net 30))
 (segment (start 110.115 96.705) (end 107.33 96.705) (width 0.35) (layer "F.Cu") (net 29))
 (segment (start 111.34 95.48) (end 110.115 96.705) (width 0.35) (layer "F.Cu") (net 29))
 (segment (start 106.025 95.4) (end 106 95.4) (width 0.35) (layer "F.Cu") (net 29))
 (segment (start 107.33 96.705) (end 106.025 95.4) (width 0.35) (layer "F.Cu") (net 29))
 (segment (start 110.115 99.245) (end 111.34 98.02) (width 0.35) (layer "F.Cu") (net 23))
 (segment (start 106 98) (end 107.245 99.245) (width 0.35) (layer "F.Cu") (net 23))
 (segment (start 107.245 99.245) (end 110.115 99.245) (width 0.35) (layer "F.Cu") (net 23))
 (segment (start 107.2 101.8) (end 110.1 101.8) (width 0.35) (layer "F.Cu") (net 24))
 (segment (start 110.1 101.8) (end 111.34 100.56) (width 0.35) (layer "F.Cu") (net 24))
 (segment (start 106 100.6) (end 107.2 101.8) (width 0.35) (layer "F.Cu") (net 24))
 (segment (start 110.115 104.325) (end 107.225 104.325) (width 0.35) (layer "F.Cu") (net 21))
 (segment (start 111.34 103.1) (end 110.115 104.325) (width 0.35) (layer "F.Cu") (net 21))
 (segment (start 107.225 104.325) (end 106 103.1) (width 0.35) (layer "F.Cu") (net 21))
 (segment (start 111.34 105.64) (end 110.08 106.9) (width 0.35) (layer "F.Cu") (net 35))
 (segment (start 110.08 106.9) (end 107.2 106.9) (width 0.35) (layer "F.Cu") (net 35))
 (segment (start 107.2 106.9) (end 106 105.7) (width 0.35) (layer "F.Cu") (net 35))
 (segment (start 106 105.7) (end 106 105.6) (width 0.35) (layer "F.Cu") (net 35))
 (segment (start 108.8 110.72) (end 108.32 111.2) (width 0.35) (layer "F.Cu") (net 34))
 (segment (start 108.32 111.2) (end 106 111.2) (width 0.35) (layer "F.Cu") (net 34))
 (segment (start 106.295 109.495) (end 106 109.2) (width 0.35) (layer "F.Cu") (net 32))
 (segment (start 111.34 110.72) (end 110.115 109.495) (width 0.35) (layer "F.Cu") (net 32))
 (segment (start 110.115 109.495) (end 106.295 109.495) (width 0.35) (layer "F.Cu") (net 32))
 (segment (start 106 113.3) (end 107.265 112.035) (width 0.35) (layer "F.Cu") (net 22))
 (segment (start 107.265 112.035) (end 110.115 112.035) (width 0.35) (layer "F.Cu") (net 22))
 (segment (start 110.115 112.035) (end 111.34 113.26) (width 0.35) (layer "F.Cu") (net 22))
 (segment (start 111.34 115.8) (end 110.04 114.5) (width 0.35) (layer "F.Cu") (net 26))
 (segment (start 107.3 114.5) (end 106 115.8) (width 0.35) (layer "F.Cu") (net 26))
 (segment (start 110.04 114.5) (end 107.3 114.5) (width 0.35) (layer "F.Cu") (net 26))
 (segment (start 99.34 113.26) (end 103.96 113.26) (width 0.35) (layer "F.Cu") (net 19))
 (segment (start 103.96 113.26) (end 104 113.3) (width 0.35) (layer "F.Cu") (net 19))
 (segment (start 99.34 115.8) (end 104 115.8) (width 0.35) (layer "F.Cu") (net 20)))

